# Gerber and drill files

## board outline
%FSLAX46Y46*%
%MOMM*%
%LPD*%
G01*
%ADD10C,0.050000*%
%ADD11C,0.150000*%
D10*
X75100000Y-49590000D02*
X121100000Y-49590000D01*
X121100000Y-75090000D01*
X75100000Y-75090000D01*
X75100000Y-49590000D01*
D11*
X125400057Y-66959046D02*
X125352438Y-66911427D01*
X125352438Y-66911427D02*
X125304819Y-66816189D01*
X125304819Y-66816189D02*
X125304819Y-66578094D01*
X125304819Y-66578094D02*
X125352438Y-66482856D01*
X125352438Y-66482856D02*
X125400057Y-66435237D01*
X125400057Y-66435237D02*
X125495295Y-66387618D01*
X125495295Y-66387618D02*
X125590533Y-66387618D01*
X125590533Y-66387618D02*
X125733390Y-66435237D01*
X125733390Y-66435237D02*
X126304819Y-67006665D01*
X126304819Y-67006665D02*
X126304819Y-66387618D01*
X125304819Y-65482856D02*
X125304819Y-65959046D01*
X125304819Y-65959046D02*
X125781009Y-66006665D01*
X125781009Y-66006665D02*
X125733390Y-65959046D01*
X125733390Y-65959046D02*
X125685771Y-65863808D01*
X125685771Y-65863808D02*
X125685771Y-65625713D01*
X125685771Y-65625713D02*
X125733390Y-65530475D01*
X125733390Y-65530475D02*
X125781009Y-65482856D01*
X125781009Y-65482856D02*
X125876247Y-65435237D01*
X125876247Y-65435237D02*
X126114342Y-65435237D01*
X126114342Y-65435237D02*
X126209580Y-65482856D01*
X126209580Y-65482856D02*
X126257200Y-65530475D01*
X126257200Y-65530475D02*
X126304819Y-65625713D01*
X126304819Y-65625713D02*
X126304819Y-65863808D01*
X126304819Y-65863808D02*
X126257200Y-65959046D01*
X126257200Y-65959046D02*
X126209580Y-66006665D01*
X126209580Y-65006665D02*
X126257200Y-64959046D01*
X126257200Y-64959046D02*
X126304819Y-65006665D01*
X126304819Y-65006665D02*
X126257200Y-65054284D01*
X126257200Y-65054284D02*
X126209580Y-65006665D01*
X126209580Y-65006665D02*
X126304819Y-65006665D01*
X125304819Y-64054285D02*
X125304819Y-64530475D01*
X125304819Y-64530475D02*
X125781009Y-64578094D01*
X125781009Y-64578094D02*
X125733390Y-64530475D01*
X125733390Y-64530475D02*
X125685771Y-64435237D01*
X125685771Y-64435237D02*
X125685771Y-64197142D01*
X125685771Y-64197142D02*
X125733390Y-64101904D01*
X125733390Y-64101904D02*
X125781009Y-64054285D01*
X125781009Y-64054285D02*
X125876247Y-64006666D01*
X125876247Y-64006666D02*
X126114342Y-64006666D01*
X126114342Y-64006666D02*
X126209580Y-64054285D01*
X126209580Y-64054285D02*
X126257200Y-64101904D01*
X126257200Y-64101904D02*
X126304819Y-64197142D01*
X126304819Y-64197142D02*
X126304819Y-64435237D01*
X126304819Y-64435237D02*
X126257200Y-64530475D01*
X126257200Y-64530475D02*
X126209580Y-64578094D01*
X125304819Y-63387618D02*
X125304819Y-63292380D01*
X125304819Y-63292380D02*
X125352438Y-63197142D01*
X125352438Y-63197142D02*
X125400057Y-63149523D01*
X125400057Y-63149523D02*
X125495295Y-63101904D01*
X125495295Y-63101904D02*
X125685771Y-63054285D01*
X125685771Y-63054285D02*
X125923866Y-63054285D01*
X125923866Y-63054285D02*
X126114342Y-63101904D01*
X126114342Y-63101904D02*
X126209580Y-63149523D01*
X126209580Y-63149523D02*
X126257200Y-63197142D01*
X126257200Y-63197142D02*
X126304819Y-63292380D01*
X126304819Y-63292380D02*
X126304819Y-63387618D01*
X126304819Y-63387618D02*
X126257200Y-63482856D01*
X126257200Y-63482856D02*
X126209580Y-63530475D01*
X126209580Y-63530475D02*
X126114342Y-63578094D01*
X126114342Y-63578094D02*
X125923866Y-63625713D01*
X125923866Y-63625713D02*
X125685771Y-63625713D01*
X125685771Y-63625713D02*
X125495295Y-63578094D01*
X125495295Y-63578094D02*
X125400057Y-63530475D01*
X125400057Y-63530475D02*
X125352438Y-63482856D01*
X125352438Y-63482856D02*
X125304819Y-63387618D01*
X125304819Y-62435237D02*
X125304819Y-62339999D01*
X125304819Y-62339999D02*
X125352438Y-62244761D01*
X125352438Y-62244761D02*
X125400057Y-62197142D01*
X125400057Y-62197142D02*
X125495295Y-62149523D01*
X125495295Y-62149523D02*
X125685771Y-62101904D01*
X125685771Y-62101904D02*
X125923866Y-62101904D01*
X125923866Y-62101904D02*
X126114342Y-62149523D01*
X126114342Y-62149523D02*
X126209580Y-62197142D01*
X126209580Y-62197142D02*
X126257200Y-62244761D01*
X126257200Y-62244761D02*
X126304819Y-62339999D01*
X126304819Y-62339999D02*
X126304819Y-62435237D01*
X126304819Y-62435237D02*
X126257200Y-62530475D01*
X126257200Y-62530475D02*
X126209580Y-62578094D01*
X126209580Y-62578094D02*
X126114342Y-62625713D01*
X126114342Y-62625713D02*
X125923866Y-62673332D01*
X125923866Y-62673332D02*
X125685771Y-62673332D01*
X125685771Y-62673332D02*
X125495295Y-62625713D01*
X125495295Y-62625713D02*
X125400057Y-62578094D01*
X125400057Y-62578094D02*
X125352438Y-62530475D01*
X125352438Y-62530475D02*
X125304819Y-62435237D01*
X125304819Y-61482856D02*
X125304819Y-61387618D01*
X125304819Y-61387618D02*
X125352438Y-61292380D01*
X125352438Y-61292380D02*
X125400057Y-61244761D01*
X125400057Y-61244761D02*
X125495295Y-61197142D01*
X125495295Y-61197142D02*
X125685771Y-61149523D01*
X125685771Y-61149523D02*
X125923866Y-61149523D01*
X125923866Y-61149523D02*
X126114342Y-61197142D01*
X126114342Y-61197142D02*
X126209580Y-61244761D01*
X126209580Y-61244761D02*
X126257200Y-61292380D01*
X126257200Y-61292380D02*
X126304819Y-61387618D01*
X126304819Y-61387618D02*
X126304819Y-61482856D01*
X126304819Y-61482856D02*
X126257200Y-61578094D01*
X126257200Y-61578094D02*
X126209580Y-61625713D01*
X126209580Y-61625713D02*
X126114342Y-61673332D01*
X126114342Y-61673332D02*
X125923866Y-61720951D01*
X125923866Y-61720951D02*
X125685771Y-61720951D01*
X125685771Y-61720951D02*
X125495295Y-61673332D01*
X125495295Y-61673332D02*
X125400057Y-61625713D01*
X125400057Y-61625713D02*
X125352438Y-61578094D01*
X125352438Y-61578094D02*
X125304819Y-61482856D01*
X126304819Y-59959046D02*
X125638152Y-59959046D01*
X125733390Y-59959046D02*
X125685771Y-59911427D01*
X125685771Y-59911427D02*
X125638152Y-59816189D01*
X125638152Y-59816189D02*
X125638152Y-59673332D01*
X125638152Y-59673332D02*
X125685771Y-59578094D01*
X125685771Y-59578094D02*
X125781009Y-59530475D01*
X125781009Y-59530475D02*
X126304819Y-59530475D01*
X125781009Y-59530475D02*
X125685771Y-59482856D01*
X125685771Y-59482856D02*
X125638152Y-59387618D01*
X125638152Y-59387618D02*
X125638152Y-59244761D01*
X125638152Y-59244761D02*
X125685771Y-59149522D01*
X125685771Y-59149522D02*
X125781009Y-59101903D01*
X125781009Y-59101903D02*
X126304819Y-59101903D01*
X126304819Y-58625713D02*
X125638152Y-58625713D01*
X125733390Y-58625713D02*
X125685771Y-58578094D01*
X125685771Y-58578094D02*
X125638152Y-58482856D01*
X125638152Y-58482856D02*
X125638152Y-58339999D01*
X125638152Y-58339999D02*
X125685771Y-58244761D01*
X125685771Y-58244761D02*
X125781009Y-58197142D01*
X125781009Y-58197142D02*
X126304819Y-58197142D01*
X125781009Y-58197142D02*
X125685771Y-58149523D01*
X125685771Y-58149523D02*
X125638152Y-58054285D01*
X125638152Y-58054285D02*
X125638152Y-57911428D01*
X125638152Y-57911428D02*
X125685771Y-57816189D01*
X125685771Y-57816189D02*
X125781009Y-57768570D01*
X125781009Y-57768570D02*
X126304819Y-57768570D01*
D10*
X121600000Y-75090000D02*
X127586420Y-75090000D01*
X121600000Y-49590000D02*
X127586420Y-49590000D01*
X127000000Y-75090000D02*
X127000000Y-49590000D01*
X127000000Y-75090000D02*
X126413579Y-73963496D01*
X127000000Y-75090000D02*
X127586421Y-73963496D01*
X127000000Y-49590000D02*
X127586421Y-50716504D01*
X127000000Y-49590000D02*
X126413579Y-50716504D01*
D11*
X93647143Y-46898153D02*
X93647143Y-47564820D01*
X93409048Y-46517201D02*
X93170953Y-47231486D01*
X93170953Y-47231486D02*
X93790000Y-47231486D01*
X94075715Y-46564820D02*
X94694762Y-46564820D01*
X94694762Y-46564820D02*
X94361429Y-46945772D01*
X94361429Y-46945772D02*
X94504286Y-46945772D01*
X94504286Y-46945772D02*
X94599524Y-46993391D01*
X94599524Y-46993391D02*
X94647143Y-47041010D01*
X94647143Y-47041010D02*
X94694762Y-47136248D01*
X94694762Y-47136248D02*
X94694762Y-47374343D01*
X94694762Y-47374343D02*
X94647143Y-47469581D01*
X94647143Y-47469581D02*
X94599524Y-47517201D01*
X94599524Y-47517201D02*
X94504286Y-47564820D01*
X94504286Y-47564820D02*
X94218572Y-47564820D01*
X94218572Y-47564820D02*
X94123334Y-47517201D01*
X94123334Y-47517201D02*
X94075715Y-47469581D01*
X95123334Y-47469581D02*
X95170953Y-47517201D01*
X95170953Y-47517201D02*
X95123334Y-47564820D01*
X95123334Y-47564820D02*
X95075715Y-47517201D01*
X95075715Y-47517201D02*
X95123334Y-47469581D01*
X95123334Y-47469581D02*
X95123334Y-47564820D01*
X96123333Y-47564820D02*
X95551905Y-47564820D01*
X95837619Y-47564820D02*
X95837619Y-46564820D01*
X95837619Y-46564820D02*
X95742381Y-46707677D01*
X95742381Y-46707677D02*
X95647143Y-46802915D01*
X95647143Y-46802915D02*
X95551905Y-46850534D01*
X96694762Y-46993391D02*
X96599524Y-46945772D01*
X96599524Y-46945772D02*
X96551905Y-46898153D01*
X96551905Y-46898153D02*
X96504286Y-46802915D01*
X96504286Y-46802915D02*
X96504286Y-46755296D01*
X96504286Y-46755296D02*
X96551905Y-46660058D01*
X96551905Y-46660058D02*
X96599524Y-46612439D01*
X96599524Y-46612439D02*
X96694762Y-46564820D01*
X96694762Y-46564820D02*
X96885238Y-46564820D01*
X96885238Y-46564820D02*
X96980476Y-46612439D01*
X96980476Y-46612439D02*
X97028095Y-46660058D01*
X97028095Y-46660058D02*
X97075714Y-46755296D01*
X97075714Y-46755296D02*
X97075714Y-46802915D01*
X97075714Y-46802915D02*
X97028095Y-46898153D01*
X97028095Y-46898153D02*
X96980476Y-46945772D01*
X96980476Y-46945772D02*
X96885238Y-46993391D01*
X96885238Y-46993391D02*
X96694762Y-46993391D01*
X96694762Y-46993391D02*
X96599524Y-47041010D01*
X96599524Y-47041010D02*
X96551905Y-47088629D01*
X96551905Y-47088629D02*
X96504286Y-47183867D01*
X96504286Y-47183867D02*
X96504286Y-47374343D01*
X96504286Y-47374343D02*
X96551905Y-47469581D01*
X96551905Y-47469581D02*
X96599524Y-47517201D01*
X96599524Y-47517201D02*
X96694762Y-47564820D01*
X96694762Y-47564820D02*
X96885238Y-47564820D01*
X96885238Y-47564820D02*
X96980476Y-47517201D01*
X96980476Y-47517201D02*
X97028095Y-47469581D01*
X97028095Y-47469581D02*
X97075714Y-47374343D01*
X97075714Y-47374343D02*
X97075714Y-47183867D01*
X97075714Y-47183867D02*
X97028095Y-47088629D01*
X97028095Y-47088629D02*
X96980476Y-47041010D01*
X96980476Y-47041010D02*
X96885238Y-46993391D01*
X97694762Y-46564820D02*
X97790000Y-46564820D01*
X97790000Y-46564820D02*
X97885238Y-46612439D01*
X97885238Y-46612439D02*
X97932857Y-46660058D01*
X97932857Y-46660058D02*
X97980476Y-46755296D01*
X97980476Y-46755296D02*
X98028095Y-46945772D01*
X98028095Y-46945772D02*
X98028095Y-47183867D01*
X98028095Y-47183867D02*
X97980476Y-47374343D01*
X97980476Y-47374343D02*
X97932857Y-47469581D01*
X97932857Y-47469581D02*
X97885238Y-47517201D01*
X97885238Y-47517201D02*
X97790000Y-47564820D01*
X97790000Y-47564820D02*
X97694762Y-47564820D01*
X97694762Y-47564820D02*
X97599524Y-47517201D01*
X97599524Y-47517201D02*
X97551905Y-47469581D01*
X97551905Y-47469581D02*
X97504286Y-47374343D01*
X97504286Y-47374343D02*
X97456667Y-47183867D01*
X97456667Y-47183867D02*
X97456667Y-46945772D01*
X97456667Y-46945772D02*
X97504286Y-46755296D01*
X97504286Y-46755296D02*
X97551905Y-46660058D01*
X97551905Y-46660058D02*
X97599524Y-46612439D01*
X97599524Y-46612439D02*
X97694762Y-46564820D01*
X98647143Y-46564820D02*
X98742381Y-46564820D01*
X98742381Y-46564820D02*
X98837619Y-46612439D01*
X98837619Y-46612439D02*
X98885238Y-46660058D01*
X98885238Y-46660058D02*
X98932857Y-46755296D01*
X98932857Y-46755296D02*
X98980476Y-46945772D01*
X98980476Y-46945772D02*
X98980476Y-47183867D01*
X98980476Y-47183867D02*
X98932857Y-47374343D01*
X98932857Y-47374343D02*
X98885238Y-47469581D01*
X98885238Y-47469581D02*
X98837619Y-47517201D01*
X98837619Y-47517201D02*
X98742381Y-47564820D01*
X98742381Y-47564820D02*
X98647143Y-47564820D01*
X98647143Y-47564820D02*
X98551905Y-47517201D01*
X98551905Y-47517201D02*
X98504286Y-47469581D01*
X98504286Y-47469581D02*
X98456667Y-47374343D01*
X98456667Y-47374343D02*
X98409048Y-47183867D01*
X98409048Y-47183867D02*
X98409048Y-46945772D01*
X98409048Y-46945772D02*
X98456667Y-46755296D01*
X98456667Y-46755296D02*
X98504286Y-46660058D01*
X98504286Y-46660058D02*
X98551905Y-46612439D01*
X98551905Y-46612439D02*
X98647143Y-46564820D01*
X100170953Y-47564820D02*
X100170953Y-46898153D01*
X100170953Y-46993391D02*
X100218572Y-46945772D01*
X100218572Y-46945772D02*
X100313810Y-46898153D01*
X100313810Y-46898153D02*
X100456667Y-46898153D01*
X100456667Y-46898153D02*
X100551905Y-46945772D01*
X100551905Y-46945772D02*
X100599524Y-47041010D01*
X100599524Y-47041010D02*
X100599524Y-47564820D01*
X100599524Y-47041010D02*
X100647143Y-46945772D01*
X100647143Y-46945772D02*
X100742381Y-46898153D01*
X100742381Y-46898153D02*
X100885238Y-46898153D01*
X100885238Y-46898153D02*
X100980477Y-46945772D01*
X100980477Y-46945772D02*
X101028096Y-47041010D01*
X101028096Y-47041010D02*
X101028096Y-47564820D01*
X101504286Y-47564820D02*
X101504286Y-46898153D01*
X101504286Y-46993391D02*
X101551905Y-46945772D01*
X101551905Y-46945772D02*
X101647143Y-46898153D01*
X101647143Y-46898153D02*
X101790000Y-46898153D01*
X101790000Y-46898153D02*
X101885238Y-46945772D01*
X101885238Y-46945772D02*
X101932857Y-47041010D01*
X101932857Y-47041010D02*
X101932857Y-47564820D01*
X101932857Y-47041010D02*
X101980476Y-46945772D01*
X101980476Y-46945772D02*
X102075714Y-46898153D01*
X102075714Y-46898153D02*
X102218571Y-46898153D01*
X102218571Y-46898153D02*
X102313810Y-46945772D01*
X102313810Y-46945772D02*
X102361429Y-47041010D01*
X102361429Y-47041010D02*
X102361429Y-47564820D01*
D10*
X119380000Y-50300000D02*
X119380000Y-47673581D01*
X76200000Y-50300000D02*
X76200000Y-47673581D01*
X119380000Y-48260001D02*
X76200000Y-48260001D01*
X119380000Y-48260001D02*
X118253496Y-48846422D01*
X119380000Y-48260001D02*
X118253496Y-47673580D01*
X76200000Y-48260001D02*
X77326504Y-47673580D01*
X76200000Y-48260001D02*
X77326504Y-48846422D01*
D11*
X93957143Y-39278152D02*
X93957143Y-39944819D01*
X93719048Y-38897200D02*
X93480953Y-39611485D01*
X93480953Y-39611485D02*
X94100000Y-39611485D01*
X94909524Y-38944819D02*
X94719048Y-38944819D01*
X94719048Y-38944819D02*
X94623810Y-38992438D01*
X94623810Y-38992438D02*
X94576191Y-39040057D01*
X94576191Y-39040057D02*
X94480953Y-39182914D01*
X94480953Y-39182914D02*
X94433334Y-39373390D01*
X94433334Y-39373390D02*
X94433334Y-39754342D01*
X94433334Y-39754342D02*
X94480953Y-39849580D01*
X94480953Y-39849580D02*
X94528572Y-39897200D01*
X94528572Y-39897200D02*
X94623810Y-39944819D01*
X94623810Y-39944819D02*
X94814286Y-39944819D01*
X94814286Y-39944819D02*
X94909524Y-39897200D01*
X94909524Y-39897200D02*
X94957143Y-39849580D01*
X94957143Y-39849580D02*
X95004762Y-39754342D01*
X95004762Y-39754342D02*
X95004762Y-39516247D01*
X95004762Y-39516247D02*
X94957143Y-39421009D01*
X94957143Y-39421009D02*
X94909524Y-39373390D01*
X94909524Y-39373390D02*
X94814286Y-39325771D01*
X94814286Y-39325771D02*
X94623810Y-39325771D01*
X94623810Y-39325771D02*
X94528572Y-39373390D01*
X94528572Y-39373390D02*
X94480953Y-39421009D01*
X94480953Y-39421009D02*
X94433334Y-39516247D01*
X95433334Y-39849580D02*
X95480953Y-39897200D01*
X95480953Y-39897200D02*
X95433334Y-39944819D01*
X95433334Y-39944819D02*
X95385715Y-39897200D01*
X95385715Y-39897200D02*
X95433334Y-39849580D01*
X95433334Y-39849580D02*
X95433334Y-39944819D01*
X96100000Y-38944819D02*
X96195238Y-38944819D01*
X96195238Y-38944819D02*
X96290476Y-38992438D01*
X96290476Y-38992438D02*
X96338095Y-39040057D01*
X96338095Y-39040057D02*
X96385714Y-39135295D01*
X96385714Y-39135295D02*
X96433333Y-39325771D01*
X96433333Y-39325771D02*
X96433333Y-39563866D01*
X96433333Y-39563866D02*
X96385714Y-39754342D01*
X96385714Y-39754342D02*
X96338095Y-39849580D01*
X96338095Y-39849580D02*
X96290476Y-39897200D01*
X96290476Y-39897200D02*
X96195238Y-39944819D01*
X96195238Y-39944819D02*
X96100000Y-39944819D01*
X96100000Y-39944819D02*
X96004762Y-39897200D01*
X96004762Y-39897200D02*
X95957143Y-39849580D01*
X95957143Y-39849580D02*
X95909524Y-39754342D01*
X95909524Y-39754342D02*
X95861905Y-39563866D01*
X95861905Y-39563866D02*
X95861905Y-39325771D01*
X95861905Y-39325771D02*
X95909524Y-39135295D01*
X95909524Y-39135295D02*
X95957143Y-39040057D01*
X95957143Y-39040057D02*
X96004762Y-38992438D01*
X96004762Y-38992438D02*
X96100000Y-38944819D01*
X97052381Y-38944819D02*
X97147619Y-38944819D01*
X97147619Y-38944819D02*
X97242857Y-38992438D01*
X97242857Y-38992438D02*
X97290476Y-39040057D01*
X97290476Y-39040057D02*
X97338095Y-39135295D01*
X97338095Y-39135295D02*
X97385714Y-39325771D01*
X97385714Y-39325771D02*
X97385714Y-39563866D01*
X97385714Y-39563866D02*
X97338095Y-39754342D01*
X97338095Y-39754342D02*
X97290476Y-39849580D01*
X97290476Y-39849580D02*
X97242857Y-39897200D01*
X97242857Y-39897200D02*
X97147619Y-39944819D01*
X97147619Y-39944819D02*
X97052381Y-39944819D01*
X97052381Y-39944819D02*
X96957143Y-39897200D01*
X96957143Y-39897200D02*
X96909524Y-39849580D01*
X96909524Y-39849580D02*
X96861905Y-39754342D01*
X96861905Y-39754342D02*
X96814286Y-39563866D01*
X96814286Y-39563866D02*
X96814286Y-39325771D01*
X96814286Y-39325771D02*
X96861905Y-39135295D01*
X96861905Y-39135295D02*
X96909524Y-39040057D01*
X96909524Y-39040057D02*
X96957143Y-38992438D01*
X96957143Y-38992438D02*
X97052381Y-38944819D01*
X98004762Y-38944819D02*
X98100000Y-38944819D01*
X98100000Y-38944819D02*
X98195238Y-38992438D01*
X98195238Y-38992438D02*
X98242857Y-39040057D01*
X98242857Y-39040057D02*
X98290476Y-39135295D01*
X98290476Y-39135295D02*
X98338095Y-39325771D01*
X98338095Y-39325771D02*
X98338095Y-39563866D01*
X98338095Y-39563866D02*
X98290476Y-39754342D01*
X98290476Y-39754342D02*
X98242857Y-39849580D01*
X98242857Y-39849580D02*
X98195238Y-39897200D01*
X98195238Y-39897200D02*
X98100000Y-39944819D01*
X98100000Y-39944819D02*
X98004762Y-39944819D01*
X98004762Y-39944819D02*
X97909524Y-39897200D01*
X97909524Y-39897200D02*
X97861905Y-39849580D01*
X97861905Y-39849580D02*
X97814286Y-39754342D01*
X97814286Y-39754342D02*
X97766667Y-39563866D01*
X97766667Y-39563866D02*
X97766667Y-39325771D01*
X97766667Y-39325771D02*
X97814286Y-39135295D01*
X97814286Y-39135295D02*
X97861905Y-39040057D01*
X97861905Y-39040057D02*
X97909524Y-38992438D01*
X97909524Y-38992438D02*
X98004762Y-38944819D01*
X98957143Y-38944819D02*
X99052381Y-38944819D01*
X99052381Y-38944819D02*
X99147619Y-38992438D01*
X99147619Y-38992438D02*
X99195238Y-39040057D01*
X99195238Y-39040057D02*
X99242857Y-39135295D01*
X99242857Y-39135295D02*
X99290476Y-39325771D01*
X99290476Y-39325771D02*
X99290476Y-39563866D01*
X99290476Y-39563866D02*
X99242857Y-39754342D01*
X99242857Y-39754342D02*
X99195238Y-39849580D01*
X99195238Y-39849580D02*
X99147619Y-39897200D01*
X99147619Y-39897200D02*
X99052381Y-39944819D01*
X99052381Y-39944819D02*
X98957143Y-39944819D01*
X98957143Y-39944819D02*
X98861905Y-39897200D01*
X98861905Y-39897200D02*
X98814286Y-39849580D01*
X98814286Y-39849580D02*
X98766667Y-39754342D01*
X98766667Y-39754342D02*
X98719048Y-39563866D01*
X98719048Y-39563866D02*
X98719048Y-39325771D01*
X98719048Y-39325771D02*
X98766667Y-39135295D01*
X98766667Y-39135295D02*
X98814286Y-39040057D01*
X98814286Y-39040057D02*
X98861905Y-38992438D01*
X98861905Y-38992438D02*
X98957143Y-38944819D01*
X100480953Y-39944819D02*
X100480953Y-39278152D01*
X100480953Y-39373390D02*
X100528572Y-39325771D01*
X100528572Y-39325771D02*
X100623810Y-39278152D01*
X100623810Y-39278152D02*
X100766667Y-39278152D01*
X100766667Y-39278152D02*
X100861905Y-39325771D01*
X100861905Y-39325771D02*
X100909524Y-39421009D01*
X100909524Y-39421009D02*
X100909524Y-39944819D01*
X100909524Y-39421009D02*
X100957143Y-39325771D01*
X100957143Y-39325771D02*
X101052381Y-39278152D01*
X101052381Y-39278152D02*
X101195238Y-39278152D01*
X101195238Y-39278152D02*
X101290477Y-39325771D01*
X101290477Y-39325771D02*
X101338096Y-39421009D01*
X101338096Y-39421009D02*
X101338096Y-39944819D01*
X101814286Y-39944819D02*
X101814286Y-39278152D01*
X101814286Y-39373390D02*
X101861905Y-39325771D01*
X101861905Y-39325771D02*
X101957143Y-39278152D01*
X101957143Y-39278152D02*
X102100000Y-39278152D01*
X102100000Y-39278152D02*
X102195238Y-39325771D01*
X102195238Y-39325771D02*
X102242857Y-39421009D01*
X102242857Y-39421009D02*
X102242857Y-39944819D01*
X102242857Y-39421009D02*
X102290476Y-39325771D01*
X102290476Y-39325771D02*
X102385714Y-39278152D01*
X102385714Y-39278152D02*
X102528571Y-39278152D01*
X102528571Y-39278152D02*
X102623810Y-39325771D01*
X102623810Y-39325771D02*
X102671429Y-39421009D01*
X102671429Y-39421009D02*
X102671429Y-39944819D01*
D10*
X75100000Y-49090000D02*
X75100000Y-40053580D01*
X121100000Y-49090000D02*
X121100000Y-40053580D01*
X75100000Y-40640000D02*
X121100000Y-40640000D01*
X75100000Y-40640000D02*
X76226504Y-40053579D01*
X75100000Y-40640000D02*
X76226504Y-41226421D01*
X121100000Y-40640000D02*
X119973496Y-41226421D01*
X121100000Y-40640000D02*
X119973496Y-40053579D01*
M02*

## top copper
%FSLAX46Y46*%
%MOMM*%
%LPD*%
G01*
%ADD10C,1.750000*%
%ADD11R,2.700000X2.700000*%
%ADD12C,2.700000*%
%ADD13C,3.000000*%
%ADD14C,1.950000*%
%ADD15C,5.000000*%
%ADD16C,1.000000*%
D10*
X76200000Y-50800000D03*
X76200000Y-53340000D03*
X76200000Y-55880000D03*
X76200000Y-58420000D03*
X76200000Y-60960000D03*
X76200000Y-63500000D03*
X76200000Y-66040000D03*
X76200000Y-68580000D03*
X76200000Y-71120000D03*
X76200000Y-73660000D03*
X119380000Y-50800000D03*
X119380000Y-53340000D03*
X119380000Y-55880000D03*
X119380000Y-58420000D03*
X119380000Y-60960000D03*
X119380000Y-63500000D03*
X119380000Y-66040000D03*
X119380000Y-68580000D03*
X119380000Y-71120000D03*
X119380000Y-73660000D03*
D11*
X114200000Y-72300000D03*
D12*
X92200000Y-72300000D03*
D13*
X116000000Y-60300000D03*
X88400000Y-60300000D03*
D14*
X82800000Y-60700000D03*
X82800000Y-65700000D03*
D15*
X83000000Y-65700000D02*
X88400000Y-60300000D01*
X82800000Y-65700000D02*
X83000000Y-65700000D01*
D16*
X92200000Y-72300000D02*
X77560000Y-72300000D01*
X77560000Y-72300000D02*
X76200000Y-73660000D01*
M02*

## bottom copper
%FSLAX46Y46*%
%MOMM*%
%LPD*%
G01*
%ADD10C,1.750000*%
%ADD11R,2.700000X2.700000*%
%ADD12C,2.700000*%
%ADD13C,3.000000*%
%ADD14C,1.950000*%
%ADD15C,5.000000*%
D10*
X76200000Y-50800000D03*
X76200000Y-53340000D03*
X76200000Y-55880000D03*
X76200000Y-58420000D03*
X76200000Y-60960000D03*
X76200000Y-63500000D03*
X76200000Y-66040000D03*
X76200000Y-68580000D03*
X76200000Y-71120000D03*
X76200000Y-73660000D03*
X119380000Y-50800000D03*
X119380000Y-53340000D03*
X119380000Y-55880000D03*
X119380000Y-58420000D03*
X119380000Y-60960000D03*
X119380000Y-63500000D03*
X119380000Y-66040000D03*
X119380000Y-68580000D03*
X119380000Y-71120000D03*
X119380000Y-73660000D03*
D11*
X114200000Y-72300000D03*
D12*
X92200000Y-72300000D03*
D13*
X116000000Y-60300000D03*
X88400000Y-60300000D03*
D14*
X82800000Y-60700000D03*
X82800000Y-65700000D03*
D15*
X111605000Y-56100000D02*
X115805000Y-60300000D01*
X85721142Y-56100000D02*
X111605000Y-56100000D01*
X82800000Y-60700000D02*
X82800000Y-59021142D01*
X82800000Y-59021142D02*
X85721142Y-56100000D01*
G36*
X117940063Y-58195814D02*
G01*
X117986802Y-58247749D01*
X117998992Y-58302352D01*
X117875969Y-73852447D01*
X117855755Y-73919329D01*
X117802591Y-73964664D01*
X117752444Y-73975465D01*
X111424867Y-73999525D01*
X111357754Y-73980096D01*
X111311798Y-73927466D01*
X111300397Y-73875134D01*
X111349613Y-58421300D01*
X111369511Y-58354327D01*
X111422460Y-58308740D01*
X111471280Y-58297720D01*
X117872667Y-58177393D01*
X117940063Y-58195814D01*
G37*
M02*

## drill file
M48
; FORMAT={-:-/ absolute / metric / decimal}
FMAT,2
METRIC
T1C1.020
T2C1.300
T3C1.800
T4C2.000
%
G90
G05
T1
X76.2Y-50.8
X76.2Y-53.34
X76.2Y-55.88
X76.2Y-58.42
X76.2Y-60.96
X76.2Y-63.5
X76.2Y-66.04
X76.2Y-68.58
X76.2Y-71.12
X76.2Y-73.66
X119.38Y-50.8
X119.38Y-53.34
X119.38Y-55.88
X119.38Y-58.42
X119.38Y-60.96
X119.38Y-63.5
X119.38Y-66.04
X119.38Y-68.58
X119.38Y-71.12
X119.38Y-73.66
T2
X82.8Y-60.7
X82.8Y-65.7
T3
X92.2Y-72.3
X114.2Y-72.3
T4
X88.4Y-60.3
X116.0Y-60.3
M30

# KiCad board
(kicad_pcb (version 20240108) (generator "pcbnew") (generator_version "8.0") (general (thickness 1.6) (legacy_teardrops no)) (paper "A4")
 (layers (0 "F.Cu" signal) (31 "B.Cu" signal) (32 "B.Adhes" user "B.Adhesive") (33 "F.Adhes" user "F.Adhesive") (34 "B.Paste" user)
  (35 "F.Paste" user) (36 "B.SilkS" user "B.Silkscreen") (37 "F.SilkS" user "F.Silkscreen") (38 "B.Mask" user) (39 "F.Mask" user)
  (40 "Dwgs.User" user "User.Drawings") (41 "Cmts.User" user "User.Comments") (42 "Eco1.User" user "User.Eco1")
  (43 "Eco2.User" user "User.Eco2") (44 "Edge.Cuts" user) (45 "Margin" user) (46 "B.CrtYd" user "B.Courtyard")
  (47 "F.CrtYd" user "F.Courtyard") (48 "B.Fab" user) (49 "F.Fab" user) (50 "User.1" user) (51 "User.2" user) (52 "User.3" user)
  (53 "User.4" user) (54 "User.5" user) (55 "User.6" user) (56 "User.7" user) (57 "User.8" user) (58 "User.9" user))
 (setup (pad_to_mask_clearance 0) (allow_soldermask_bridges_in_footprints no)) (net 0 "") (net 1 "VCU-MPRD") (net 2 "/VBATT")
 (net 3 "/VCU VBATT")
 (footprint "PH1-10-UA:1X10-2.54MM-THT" (layer "F.Cu") (at 76.2 50.8 -90)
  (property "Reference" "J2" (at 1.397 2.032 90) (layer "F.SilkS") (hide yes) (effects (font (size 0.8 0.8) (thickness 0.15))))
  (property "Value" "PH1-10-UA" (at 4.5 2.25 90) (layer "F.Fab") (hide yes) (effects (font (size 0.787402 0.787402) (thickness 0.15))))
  (pad "1" thru_hole circle (at 0 0 270) (size 1.75 1.75) (drill 1.02) (layers "*.Cu" "*.Mask") (remove_unused_layers no)
   (solder_mask_margin 0.102))
  (pad "2" thru_hole circle (at 2.54 0 270) (size 1.75 1.75) (drill 1.02) (layers "*.Cu" "*.Mask") (remove_unused_layers no)
   (solder_mask_margin 0.102))
  (pad "3" thru_hole circle (at 5.08 0 270) (size 1.75 1.75) (drill 1.02) (layers "*.Cu" "*.Mask") (remove_unused_layers no)
   (solder_mask_margin 0.102))
  (pad "4" thru_hole circle (at 7.62 0 270) (size 1.75 1.75) (drill 1.02) (layers "*.Cu" "*.Mask") (remove_unused_layers no)
   (solder_mask_margin 0.102))
  (pad "5" thru_hole circle (at 10.16 0 270) (size 1.75 1.75) (drill 1.02) (layers "*.Cu" "*.Mask") (remove_unused_layers no)
   (solder_mask_margin 0.102))
  (pad "6" thru_hole circle (at 12.7 0 270) (size 1.75 1.75) (drill 1.02) (layers "*.Cu" "*.Mask") (remove_unused_layers no)
   (solder_mask_margin 0.102))
  (pad "7" thru_hole circle (at 15.24 0 270) (size 1.75 1.75) (drill 1.02) (layers "*.Cu" "*.Mask") (remove_unused_layers no)
   (solder_mask_margin 0.102))
  (pad "8" thru_hole circle (at 17.78 0 270) (size 1.75 1.75) (drill 1.02) (layers "*.Cu" "*.Mask") (remove_unused_layers no)
   (solder_mask_margin 0.102))
  (pad "9" thru_hole circle (at 20.32 0 270) (size 1.75 1.75) (drill 1.02) (layers "*.Cu" "*.Mask") (remove_unused_layers no)
   (solder_mask_margin 0.102))
  (pad "10" thru_hole circle (at 22.86 0 270) (size 1.75 1.75) (drill 1.02) (layers "*.Cu" "*.Mask") (remove_unused_layers no)
   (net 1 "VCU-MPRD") (solder_mask_margin 0.102)))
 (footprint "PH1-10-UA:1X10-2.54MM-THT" (layer "F.Cu") (at 119.38 50.8 -90)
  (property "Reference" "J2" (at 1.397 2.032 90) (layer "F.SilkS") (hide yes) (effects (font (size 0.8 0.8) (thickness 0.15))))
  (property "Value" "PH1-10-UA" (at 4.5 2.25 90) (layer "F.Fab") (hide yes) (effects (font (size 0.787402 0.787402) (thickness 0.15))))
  (pad "1" thru_hole circle (at 0 0 270) (size 1.75 1.75) (drill 1.02) (layers "*.Cu" "*.Mask") (remove_unused_layers no)
   (solder_mask_margin 0.102))
  (pad "2" thru_hole circle (at 2.54 0 270) (size 1.75 1.75) (drill 1.02) (layers "*.Cu" "*.Mask") (remove_unused_layers no)
   (solder_mask_margin 0.102))
  (pad "3" thru_hole circle (at 5.08 0 270) (size 1.75 1.75) (drill 1.02) (layers "*.Cu" "*.Mask") (remove_unused_layers no)
   (solder_mask_margin 0.102))
  (pad "4" thru_hole circle (at 7.62 0 270) (size 1.75 1.75) (drill 1.02) (layers "*.Cu" "*.Mask") (remove_unused_layers no)
   (solder_mask_margin 0.102))
  (pad "5" thru_hole circle (at 10.16 0 270) (size 1.75 1.75) (drill 1.02) (layers "*.Cu" "*.Mask") (remove_unused_layers no)
   (solder_mask_margin 0.102))
  (pad "6" thru_hole circle (at 12.7 0 270) (size 1.75 1.75) (drill 1.02) (layers "*.Cu" "*.Mask") (remove_unused_layers no)
   (solder_mask_margin 0.102))
  (pad "7" thru_hole circle (at 15.24 0 270) (size 1.75 1.75) (drill 1.02) (layers "*.Cu" "*.Mask") (remove_unused_layers no)
   (solder_mask_margin 0.102))
  (pad "8" thru_hole circle (at 17.78 0 270) (size 1.75 1.75) (drill 1.02) (layers "*.Cu" "*.Mask") (remove_unused_layers no)
   (solder_mask_margin 0.102))
  (pad "9" thru_hole circle (at 20.32 0 270) (size 1.75 1.75) (drill 1.02) (layers "*.Cu" "*.Mask") (remove_unused_layers no)
   (solder_mask_margin 0.102))
  (pad "10" thru_hole circle (at 22.86 0 270) (size 1.75 1.75) (drill 1.02) (layers "*.Cu" "*.Mask") (remove_unused_layers no)
   (solder_mask_margin 0.102)))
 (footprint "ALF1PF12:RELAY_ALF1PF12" (layer "F.Cu") (at 102.2 66.3 180)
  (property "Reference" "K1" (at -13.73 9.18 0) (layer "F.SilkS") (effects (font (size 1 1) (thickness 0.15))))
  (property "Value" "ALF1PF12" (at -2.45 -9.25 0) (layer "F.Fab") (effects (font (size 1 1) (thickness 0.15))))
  (pad "1" thru_hole rect (at -12 -6 180) (size 2.7 2.7) (drill 1.8) (layers "*.Cu" "*.Mask") (remove_unused_layers no) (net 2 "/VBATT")
   (solder_mask_margin 0.102))
  (pad "2" thru_hole circle (at 10 -6 180) (size 2.7 2.7) (drill 1.8) (layers "*.Cu" "*.Mask") (remove_unused_layers no) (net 1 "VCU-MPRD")
   (solder_mask_margin 0.102))
  (pad "3" thru_hole circle (at -13.8 6 180) (size 3 3) (drill 2) (layers "*.Cu" "*.Mask") (remove_unused_layers no) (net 2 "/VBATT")
   (solder_mask_margin 0.102))
  (pad "4" thru_hole circle (at 13.8 6 180) (size 3 3) (drill 2) (layers "*.Cu" "*.Mask") (remove_unused_layers no) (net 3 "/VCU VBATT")
   (solder_mask_margin 0.102)))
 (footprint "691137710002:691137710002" (layer "F.Cu") (at 82.8 63.2 -90)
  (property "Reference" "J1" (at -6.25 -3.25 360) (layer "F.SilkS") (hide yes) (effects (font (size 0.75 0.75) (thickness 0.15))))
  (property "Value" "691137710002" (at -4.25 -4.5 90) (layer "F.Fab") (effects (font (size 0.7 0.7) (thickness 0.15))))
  (pad "1" thru_hole circle (at -2.5 0 270) (size 1.95 1.95) (drill 1.3) (layers "*.Cu" "*.Mask") (remove_unused_layers no) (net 2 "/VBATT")
   (solder_mask_margin 0.102))
  (pad "2" thru_hole circle (at 2.5 0 270) (size 1.95 1.95) (drill 1.3) (layers "*.Cu" "*.Mask") (remove_unused_layers no)
   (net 3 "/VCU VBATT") (solder_mask_margin 0.102)))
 (gr_rect (start 75.1 49.59) (end 121.1 75.09) (stroke (width 0.05) (type default)) (fill none) (layer "Edge.Cuts"))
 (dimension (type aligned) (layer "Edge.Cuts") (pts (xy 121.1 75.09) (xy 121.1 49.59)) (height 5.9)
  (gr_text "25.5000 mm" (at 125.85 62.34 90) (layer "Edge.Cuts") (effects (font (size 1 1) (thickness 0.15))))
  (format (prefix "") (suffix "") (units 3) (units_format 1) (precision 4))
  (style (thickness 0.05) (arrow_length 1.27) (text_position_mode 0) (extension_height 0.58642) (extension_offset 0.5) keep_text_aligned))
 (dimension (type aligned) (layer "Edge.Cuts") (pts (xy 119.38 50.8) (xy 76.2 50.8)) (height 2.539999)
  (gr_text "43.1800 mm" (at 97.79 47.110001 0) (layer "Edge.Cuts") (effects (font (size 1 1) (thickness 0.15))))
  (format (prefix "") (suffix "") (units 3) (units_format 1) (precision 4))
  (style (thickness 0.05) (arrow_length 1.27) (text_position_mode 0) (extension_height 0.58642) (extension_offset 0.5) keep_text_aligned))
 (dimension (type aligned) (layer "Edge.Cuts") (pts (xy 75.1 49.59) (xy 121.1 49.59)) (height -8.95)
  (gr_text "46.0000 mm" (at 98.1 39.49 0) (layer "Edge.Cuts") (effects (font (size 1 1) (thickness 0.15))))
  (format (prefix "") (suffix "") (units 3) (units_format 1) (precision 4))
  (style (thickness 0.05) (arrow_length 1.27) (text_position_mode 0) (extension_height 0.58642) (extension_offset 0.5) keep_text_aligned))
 (segment (start 111.605 56.1) (end 115.805 60.3) (width 5) (layer "B.Cu") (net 2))
 (segment (start 85.721142 56.1) (end 111.605 56.1) (width 5) (layer "B.Cu") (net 2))
 (segment (start 82.8 60.7) (end 82.8 59.021142) (width 5) (layer "B.Cu") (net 2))
 (segment (start 82.8 59.021142) (end 85.721142 56.1) (width 5) (layer "B.Cu") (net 2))
 (segment (start 83 65.7) (end 88.4 60.3) (width 5) (layer "F.Cu") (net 3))
 (segment (start 82.8 65.7) (end 83 65.7) (width 5) (layer "F.Cu") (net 3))
 (segment (start 92.2 72.3) (end 77.56 72.3) (width 1) (layer "F.Cu") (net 1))
 (segment (start 77.56 72.3) (end 76.2 73.66) (width 1) (layer "F.Cu") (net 1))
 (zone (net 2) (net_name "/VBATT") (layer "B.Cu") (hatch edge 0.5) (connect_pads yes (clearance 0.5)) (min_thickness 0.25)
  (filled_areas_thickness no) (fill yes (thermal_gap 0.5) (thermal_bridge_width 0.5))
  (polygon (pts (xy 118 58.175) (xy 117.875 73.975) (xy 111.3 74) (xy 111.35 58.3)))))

